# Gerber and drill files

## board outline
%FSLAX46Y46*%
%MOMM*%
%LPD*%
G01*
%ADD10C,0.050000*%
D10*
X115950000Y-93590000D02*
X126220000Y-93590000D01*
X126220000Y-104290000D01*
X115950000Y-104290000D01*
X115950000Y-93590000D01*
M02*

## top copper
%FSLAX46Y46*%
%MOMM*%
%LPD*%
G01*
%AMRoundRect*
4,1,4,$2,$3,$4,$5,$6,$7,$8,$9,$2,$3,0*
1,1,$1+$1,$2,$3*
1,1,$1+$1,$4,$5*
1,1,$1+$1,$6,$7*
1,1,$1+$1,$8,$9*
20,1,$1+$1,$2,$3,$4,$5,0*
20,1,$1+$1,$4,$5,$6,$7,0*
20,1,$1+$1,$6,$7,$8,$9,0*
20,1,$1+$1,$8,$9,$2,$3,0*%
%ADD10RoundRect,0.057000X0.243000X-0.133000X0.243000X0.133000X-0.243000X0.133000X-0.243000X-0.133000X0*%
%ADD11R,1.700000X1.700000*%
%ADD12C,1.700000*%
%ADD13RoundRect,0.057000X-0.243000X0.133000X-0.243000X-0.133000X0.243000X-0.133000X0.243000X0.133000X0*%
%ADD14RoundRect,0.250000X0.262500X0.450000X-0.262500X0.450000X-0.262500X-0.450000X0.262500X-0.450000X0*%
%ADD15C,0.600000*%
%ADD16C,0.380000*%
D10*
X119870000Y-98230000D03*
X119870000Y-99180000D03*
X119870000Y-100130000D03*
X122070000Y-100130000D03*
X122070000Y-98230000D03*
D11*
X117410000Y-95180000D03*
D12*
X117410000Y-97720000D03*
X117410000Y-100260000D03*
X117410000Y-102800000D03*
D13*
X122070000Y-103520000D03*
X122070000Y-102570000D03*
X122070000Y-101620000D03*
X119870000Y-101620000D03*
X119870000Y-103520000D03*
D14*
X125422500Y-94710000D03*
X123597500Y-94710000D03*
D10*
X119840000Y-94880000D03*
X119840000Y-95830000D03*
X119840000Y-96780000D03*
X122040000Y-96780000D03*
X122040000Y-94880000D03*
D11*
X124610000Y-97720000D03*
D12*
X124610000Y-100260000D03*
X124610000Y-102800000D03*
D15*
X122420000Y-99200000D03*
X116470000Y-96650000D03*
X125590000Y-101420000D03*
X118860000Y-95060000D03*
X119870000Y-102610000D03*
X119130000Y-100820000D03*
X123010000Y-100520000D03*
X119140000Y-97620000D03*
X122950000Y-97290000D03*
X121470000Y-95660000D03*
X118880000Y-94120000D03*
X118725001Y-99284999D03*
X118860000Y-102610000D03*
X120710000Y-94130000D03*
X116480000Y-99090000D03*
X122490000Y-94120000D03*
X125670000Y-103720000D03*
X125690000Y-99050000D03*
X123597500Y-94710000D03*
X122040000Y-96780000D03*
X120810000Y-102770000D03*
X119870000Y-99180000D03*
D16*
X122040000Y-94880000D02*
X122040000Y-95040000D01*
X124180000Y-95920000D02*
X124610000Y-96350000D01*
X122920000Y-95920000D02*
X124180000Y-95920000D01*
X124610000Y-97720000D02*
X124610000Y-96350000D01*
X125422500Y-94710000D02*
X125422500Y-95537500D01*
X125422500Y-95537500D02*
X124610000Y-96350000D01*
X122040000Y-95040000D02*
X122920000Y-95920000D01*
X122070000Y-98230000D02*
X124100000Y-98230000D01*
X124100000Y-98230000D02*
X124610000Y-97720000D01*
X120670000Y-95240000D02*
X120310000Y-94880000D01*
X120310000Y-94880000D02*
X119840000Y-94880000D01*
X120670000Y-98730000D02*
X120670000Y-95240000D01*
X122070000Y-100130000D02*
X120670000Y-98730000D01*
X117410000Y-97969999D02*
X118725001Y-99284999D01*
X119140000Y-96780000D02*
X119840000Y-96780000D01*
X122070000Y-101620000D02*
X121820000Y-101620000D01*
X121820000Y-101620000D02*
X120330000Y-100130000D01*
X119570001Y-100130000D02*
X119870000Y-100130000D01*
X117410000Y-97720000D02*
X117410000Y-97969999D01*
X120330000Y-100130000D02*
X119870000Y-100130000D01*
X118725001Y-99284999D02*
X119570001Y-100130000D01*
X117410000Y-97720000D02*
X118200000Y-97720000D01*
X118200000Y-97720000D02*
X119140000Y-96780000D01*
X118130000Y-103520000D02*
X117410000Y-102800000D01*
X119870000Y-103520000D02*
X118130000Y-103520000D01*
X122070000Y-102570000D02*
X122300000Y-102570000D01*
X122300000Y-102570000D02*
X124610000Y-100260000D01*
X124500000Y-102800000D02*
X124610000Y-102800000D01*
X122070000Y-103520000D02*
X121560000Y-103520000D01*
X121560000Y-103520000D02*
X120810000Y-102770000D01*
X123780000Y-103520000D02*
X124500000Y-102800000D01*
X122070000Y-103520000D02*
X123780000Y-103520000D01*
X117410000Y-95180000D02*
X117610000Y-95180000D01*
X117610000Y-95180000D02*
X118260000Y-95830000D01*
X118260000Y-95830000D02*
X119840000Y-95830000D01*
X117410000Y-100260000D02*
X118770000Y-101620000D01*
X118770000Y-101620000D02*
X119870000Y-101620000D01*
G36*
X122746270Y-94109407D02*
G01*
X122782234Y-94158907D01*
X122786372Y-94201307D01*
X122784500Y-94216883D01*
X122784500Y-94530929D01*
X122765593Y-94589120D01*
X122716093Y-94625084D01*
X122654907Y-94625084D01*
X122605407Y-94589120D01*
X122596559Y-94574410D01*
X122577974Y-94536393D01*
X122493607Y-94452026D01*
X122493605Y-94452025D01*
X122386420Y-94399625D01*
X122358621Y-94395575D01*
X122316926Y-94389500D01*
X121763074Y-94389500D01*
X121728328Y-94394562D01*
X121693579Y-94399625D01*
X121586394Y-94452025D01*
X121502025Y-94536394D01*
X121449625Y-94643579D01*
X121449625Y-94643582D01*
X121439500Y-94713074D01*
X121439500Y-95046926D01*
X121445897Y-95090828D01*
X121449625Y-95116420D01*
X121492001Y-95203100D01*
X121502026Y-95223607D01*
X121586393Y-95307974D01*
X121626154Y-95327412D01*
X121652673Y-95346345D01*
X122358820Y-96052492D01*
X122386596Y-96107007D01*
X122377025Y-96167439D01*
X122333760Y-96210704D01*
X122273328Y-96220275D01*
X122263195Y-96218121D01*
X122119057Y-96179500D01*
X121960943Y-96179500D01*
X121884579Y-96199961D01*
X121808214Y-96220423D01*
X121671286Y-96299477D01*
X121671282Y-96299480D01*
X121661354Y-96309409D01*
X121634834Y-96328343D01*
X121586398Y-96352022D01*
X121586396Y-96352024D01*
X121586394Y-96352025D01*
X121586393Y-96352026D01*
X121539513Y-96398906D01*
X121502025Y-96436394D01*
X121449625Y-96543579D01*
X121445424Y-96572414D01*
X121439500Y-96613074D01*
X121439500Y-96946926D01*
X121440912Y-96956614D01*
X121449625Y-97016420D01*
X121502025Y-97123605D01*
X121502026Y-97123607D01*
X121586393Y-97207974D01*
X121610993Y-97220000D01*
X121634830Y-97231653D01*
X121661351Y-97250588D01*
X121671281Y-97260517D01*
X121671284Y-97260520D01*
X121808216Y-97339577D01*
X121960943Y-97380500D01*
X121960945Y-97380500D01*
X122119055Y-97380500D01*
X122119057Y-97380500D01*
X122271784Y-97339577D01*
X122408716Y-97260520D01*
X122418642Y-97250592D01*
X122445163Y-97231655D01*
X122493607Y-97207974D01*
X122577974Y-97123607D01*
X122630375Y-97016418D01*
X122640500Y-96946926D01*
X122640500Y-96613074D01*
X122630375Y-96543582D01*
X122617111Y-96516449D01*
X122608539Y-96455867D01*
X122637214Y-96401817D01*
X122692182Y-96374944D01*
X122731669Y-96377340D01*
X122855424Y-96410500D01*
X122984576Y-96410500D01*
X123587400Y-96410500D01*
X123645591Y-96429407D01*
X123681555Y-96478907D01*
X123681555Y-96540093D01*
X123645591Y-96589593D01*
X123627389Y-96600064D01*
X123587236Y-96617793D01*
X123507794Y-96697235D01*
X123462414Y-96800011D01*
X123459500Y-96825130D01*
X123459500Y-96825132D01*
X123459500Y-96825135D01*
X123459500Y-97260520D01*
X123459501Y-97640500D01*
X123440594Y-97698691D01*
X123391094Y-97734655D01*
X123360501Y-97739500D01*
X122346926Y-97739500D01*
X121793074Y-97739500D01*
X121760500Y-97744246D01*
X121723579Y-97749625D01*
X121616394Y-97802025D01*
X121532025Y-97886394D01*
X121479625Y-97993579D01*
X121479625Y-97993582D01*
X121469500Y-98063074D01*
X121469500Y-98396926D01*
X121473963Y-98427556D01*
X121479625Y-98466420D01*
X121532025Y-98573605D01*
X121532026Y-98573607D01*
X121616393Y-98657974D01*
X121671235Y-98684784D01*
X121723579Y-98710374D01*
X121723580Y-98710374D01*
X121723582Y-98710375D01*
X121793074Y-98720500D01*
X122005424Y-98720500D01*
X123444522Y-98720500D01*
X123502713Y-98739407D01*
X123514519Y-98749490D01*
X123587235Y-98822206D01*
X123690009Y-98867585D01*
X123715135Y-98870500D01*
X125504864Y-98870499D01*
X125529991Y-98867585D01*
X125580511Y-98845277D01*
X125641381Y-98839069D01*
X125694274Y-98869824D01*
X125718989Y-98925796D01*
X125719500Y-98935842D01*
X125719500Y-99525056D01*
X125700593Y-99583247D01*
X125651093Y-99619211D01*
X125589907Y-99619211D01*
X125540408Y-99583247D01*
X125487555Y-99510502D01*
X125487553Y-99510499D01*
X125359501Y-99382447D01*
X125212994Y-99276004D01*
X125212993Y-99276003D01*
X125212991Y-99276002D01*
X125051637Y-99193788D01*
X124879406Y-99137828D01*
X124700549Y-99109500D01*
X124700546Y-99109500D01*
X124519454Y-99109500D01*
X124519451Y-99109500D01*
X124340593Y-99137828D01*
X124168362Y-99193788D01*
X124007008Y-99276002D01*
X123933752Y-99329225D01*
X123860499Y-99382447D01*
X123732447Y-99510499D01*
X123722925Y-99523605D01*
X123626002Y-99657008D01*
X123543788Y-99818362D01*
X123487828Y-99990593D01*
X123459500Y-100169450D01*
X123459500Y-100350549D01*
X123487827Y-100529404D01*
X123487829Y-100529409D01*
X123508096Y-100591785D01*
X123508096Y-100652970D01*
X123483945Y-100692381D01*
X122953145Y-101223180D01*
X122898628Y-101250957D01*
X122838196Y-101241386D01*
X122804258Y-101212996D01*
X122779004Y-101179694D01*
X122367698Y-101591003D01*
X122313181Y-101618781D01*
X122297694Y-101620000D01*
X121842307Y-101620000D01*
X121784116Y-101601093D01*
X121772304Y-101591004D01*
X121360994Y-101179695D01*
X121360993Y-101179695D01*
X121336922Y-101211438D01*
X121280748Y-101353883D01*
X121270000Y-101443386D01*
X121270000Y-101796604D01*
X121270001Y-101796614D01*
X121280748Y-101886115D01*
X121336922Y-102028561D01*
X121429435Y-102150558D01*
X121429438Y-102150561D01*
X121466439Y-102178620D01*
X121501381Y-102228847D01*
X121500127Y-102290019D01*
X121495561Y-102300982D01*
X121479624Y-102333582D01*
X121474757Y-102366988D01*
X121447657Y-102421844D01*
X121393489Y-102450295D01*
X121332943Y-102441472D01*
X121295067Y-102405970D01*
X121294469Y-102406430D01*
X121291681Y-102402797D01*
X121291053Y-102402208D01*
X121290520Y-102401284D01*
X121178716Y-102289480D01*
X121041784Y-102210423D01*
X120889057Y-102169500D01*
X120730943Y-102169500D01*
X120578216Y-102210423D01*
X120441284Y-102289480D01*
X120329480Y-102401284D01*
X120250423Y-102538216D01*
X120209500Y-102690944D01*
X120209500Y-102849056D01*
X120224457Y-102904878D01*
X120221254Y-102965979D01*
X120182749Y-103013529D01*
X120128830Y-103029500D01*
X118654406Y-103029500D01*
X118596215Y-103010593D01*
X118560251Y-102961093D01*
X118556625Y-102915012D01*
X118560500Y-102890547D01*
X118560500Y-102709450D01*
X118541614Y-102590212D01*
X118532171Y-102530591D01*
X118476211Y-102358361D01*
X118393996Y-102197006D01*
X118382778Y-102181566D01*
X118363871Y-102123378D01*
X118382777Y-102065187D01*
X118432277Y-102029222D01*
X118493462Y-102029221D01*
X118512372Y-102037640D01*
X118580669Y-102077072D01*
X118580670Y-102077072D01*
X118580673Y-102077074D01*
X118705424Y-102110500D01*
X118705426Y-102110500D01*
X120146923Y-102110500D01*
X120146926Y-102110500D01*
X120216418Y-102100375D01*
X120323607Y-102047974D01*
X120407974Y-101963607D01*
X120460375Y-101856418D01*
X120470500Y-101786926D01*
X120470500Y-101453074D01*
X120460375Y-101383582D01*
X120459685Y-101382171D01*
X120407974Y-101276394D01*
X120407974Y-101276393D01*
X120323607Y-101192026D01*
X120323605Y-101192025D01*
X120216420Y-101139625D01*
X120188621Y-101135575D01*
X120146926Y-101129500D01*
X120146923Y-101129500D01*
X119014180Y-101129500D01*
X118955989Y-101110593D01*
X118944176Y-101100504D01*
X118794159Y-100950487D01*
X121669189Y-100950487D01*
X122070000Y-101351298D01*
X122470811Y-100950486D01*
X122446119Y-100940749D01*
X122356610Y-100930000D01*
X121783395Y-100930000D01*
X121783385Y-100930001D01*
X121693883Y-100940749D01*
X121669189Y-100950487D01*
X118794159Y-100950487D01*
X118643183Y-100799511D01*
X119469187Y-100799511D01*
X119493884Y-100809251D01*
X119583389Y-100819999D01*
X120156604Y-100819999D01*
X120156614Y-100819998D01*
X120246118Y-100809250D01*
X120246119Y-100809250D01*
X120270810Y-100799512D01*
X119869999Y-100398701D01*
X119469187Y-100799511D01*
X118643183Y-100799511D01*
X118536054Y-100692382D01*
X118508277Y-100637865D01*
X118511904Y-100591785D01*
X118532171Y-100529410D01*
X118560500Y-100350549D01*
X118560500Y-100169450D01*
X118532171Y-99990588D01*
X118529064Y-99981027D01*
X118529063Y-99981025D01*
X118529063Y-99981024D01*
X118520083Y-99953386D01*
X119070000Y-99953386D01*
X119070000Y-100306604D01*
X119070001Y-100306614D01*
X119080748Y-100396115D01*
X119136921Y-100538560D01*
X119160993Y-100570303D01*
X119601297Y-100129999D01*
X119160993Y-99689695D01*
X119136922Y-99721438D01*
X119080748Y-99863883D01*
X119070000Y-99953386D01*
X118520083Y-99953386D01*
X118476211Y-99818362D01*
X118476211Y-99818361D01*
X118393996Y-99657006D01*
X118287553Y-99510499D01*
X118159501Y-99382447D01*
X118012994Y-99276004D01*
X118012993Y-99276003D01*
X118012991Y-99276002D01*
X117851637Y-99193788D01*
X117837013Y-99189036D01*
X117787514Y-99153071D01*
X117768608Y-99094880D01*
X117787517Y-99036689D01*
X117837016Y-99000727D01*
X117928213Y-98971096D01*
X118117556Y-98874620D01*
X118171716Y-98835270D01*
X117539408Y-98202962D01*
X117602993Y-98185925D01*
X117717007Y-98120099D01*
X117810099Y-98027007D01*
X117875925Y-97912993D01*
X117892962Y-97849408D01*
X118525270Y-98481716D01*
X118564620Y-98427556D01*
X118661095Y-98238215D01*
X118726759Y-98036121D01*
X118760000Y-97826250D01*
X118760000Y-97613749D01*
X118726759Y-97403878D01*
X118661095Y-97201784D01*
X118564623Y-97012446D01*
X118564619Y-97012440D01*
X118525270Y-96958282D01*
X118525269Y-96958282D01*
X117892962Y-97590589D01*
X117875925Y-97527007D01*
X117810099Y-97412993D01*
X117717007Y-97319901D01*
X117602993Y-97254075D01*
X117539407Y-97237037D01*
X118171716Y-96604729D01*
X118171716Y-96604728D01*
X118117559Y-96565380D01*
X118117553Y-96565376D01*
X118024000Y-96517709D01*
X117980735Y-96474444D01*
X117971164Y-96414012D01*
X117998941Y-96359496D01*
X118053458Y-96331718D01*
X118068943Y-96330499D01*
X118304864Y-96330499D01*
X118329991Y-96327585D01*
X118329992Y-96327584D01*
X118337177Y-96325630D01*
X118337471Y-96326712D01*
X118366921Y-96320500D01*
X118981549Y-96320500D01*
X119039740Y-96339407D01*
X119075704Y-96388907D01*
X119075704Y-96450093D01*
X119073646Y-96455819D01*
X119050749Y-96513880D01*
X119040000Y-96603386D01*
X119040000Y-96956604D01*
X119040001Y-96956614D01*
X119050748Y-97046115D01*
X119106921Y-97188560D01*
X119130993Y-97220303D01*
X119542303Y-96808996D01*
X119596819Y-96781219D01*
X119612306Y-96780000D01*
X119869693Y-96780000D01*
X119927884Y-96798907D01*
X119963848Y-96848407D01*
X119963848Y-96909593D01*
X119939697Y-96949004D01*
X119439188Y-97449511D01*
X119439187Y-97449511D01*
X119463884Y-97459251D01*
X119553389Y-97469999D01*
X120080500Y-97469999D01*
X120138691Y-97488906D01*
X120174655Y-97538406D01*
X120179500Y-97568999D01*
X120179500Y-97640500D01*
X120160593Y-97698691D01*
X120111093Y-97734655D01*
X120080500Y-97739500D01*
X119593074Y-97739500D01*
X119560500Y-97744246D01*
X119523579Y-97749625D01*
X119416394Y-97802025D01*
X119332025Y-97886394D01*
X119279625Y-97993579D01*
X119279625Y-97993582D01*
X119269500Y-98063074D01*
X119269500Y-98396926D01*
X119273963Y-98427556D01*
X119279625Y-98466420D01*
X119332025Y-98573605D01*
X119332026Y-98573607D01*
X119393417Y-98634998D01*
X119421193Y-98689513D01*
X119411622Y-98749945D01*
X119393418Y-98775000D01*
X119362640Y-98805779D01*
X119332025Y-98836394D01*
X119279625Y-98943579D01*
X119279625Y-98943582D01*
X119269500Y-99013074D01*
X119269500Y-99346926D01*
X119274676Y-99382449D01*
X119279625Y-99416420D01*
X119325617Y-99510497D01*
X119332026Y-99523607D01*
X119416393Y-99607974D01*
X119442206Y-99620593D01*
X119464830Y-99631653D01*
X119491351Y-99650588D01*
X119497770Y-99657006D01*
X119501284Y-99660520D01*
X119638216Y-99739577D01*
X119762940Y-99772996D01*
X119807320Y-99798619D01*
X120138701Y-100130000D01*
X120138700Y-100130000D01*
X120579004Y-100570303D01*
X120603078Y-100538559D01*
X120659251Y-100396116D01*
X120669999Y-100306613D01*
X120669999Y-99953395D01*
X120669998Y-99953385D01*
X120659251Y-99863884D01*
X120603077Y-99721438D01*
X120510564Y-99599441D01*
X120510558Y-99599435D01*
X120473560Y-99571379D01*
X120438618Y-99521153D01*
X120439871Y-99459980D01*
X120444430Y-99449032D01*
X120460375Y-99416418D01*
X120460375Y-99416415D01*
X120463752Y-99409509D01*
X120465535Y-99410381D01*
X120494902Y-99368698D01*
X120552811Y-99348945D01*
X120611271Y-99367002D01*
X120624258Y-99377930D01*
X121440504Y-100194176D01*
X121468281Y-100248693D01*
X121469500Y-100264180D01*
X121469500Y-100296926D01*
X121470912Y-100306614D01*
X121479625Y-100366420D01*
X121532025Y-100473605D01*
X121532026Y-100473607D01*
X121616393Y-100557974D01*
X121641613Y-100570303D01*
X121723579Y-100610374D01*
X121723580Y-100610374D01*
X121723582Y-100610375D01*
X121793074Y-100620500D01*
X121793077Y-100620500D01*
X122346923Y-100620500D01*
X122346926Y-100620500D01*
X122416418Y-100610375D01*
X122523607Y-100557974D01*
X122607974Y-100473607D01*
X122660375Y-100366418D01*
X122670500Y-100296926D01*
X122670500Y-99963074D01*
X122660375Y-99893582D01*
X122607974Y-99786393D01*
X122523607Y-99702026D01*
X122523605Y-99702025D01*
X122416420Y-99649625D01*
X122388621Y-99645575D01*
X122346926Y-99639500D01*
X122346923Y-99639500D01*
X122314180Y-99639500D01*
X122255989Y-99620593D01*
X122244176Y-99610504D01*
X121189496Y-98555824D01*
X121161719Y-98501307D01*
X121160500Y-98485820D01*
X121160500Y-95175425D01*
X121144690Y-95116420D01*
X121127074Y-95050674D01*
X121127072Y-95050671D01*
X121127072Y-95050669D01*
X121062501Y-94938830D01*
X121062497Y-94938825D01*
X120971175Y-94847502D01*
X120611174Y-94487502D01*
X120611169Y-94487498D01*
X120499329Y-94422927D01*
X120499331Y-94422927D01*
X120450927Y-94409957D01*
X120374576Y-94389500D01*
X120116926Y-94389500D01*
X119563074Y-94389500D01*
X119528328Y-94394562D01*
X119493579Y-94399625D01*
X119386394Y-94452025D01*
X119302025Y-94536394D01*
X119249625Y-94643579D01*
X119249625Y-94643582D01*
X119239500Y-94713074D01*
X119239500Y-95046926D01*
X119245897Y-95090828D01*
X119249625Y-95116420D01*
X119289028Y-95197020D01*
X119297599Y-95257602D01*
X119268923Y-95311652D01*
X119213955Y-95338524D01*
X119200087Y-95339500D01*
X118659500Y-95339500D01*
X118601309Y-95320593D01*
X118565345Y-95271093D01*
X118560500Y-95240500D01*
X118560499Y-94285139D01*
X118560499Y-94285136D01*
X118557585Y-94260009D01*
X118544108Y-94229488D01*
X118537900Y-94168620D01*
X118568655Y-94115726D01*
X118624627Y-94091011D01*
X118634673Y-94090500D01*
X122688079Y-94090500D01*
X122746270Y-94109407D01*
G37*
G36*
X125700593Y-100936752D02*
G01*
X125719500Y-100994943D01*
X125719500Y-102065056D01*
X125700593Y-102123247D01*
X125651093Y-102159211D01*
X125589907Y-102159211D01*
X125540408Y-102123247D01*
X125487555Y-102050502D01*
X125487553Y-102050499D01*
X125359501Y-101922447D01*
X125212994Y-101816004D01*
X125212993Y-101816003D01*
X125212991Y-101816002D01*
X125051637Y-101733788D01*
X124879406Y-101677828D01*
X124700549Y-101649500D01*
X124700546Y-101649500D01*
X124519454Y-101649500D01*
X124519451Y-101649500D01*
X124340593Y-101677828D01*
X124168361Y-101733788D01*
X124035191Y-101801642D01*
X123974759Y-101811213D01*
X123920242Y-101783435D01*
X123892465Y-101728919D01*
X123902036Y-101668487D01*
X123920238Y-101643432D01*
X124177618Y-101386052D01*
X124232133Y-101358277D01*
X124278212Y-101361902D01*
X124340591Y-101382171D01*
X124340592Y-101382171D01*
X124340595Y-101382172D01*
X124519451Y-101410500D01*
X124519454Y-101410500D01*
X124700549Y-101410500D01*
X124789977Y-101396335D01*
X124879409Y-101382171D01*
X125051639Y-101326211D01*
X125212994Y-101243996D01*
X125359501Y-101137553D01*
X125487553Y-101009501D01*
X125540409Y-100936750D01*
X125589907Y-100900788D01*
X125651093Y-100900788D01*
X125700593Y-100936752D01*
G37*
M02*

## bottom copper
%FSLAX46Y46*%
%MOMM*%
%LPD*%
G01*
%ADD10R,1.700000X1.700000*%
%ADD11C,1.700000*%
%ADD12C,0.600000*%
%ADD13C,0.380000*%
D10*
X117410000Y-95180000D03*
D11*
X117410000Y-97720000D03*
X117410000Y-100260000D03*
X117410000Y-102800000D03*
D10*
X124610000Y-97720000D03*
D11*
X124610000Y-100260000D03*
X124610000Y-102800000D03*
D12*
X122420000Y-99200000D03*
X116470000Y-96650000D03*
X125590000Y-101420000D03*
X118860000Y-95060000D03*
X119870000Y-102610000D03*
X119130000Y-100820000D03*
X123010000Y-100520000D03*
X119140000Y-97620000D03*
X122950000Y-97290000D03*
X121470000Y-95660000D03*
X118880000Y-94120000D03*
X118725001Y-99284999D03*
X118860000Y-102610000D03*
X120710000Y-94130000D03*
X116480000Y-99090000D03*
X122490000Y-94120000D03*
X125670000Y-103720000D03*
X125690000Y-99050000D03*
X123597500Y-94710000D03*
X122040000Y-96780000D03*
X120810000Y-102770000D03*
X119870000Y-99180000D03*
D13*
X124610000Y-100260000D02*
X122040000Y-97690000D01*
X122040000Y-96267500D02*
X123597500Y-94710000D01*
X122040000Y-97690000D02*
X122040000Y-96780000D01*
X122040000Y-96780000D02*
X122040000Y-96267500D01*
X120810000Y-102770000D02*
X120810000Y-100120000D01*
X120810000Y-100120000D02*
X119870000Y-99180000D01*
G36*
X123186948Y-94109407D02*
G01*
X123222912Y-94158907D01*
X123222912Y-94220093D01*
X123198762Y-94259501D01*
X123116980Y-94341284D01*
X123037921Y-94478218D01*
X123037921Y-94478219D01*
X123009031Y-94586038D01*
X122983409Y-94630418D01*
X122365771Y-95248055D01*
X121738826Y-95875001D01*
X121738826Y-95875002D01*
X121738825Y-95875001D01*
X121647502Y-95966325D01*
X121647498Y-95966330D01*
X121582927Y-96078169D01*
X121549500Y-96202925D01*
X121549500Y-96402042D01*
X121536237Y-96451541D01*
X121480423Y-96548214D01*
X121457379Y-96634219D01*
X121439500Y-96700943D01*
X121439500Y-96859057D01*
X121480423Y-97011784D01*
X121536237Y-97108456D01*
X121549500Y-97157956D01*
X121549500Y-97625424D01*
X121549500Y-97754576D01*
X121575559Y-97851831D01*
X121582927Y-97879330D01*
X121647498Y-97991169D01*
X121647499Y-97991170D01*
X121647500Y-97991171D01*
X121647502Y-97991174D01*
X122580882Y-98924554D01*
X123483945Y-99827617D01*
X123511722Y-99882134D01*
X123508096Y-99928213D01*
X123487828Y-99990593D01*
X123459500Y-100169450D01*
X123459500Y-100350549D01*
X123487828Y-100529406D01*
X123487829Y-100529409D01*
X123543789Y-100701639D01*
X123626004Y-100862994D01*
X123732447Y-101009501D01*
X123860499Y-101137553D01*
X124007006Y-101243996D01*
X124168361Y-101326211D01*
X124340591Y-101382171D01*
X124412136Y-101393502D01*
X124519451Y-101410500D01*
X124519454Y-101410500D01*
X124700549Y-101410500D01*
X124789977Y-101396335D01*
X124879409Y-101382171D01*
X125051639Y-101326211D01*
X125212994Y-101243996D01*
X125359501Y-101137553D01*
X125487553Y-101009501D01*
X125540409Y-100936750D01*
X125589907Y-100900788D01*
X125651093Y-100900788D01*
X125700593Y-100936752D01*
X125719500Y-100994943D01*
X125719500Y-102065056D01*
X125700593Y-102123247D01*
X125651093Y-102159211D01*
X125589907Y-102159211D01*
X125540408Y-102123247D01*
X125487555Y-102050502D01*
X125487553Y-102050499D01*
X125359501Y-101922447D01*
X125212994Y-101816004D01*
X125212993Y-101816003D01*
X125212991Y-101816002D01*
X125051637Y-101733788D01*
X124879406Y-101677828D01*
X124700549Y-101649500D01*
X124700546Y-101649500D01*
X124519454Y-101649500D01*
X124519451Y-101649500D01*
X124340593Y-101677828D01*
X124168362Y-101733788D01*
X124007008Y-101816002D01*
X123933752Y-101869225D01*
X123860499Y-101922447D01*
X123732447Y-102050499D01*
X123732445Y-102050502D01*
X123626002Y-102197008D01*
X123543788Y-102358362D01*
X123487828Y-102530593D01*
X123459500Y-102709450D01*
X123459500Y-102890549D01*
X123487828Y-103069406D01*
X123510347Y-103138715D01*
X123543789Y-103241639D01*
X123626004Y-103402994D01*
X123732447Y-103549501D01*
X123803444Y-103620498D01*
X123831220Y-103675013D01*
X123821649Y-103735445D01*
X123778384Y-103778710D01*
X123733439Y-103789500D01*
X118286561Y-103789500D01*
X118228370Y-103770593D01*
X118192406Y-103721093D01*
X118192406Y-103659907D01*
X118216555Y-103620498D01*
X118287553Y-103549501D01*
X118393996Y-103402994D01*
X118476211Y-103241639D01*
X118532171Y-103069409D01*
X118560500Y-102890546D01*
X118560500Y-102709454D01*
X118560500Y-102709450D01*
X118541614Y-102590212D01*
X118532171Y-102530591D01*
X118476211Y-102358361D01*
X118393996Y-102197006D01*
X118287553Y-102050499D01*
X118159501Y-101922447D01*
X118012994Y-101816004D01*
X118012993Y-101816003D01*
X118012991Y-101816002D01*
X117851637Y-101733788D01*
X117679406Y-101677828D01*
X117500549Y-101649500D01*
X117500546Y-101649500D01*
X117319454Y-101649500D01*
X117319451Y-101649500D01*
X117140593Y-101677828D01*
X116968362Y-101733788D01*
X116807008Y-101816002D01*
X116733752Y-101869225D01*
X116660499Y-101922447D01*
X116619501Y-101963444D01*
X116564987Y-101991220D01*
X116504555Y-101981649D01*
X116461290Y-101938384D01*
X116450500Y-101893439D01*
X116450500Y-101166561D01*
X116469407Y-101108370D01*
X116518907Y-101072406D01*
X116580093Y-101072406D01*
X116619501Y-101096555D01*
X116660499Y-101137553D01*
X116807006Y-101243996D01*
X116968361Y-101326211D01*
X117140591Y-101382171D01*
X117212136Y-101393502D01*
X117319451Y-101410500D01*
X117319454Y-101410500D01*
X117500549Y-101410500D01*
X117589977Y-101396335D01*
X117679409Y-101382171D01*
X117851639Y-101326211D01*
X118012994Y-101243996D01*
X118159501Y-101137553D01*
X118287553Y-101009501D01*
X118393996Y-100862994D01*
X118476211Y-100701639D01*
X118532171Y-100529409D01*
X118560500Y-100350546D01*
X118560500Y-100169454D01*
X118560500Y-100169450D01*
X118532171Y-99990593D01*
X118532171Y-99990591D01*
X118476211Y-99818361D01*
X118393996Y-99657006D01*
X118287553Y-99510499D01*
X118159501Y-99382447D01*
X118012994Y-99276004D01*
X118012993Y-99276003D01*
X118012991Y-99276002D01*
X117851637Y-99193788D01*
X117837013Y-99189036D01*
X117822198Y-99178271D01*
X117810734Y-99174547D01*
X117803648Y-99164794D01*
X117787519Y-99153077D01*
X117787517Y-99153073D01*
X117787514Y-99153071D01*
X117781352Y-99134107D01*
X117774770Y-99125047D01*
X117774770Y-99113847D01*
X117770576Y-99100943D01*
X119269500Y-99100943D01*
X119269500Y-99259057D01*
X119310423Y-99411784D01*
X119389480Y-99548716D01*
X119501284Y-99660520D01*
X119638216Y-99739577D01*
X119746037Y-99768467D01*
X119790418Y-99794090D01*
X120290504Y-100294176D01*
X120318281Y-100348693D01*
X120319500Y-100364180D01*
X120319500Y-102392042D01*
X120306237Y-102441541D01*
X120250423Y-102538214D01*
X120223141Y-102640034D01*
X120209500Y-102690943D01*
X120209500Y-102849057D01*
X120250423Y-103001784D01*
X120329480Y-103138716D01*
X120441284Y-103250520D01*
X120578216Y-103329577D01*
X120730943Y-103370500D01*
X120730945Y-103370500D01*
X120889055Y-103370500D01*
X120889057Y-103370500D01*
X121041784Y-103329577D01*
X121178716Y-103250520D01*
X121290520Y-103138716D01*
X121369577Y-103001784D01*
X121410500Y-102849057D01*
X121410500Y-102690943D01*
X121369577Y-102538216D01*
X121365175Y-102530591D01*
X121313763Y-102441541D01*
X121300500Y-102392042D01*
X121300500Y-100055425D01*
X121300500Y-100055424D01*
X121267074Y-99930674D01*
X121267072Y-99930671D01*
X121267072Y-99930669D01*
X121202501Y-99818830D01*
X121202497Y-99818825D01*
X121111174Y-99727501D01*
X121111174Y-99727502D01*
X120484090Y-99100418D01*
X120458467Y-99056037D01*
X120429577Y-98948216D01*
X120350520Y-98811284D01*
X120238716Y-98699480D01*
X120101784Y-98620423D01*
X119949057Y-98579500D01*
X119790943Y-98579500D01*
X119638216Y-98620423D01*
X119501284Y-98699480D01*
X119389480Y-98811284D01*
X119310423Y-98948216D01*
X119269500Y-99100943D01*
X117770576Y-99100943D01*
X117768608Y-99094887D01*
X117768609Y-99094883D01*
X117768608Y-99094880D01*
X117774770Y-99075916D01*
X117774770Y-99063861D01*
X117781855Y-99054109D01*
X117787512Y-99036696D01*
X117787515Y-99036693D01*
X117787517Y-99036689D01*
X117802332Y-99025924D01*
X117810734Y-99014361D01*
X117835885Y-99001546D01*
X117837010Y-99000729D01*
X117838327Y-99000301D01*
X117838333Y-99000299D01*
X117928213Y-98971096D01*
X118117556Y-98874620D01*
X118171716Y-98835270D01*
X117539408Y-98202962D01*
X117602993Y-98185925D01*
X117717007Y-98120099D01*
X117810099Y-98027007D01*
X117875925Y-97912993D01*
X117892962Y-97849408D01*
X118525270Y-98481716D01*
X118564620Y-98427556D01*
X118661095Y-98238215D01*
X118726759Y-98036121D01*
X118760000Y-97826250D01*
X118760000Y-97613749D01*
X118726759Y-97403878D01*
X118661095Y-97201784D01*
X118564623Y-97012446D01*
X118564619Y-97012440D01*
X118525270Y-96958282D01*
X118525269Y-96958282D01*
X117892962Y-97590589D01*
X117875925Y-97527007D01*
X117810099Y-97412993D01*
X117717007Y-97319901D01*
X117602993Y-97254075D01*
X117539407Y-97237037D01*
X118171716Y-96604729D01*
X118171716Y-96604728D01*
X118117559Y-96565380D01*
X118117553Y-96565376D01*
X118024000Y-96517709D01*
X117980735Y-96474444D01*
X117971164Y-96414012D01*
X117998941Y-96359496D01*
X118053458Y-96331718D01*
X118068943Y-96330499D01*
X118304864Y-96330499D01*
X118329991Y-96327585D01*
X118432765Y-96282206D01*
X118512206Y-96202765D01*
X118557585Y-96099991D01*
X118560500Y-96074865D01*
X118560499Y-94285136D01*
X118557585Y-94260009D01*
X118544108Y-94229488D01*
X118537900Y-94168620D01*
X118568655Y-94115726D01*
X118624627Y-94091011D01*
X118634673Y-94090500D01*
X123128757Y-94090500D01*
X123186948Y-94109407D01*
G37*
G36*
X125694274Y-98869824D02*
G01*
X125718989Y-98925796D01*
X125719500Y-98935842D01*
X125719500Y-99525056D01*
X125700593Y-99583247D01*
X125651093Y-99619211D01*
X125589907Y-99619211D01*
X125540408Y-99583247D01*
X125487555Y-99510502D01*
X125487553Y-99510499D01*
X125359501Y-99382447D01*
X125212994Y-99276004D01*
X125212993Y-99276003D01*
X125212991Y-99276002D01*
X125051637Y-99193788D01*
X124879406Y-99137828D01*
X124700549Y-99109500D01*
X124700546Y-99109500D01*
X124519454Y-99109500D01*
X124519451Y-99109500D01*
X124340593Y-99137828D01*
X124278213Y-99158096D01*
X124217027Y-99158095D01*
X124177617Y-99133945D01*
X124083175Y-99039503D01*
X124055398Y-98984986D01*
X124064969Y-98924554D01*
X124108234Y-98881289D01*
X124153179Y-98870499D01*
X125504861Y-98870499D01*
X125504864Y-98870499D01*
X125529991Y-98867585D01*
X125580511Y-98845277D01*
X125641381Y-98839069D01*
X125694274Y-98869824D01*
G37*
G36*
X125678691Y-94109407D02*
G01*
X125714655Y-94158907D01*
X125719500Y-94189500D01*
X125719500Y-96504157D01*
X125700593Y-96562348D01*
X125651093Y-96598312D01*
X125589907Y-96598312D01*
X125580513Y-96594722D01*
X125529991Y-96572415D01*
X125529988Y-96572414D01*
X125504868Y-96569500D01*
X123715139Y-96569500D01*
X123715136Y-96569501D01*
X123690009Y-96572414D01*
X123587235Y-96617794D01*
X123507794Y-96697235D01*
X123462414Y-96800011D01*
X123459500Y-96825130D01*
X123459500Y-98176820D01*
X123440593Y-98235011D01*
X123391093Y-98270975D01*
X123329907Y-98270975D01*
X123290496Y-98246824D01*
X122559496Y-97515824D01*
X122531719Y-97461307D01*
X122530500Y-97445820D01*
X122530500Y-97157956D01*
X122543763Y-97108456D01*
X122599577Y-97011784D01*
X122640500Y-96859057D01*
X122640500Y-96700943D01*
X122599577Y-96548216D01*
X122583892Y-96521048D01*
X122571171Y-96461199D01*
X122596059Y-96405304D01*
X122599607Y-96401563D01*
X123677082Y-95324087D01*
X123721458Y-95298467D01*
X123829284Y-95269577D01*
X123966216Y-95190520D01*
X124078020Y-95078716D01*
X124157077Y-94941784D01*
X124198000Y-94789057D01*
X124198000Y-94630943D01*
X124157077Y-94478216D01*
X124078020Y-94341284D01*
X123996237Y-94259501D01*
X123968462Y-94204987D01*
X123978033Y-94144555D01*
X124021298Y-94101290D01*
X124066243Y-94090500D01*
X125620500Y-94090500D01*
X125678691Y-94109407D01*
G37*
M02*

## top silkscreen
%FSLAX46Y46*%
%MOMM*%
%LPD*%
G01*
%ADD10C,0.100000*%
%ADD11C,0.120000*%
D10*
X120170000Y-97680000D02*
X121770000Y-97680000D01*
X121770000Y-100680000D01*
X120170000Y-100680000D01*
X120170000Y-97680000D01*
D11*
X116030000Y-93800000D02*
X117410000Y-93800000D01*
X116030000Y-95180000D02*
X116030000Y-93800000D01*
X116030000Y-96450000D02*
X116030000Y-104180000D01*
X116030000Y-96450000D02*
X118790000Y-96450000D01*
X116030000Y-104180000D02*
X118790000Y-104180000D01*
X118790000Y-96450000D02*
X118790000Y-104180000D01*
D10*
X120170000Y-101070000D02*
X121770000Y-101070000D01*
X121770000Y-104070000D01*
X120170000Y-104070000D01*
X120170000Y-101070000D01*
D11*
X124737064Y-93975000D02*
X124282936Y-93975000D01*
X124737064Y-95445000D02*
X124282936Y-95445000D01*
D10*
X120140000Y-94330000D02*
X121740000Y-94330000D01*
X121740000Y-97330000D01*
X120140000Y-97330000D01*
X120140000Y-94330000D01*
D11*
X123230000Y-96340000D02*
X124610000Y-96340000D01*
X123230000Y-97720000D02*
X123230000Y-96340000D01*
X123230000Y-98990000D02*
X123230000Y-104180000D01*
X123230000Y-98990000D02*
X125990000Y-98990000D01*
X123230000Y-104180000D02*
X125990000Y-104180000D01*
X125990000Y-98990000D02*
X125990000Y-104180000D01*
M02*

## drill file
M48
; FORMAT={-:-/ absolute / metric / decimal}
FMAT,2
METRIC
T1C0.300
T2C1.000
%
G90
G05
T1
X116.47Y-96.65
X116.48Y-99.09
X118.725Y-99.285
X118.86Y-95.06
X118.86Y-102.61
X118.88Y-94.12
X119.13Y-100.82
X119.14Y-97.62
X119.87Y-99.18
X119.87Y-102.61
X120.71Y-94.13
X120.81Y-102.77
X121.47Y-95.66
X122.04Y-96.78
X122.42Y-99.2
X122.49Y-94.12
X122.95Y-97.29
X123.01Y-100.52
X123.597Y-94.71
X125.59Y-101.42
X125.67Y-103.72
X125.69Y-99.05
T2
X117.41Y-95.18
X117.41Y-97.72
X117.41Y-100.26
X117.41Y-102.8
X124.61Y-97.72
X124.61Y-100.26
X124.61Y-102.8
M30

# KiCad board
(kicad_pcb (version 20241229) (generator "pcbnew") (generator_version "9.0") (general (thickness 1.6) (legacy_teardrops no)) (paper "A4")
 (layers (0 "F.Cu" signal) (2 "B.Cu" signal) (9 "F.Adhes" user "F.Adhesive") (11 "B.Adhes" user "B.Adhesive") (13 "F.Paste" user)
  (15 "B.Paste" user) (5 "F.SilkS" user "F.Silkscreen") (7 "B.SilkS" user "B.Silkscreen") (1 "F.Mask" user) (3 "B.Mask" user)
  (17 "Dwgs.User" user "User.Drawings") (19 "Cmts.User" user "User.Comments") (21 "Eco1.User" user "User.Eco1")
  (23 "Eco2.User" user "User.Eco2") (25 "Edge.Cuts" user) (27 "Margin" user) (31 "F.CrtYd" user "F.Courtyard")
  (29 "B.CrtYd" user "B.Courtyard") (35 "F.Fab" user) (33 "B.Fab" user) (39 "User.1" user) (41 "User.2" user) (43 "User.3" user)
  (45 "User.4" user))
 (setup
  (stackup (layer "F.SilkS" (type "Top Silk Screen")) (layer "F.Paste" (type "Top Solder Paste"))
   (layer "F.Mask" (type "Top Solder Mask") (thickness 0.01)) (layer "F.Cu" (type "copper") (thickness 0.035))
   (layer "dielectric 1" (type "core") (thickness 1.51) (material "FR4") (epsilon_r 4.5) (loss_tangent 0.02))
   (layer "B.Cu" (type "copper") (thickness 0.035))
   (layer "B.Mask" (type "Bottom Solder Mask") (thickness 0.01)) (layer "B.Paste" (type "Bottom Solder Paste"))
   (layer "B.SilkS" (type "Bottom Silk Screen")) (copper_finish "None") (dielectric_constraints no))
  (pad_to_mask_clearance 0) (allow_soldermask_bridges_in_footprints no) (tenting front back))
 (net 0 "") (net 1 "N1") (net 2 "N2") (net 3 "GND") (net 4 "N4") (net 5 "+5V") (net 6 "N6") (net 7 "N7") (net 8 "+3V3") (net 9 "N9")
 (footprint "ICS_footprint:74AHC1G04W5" (layer "F.Cu") (at 120.97 99.18 90)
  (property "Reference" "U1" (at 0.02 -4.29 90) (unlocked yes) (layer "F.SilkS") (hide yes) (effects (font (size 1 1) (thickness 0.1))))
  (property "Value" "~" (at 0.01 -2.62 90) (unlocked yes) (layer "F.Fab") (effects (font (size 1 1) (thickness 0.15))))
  (fp_rect (start -1.5 -0.8) (end 1.5 0.8) (stroke (width 0.1) (type solid)) (fill no) (layer "F.SilkS"))
  (pad "1" smd roundrect (at 0.95 -1.1 90) (size 0.38 0.6) (layers "F.Cu" "F.Mask" "F.Paste") (roundrect_rratio 0.15) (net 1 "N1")
   (thermal_bridge_angle 45))
  (pad "2" smd roundrect (at 0 -1.1 90) (size 0.38 0.6) (layers "F.Cu" "F.Mask" "F.Paste") (roundrect_rratio 0.15) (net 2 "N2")
   (thermal_bridge_angle 45))
  (pad "3" smd roundrect (at -0.95 -1.1 90) (size 0.38 0.6) (layers "F.Cu" "F.Mask" "F.Paste") (roundrect_rratio 0.15) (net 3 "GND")
   (thermal_bridge_angle 45))
  (pad "4" smd roundrect (at -0.95 1.1 90) (size 0.38 0.6) (layers "F.Cu" "F.Mask" "F.Paste") (roundrect_rratio 0.15) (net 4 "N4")
   (thermal_bridge_angle 45))
  (pad "5" smd roundrect (at 0.95 1.1 90) (size 0.38 0.6) (layers "F.Cu" "F.Mask" "F.Paste") (roundrect_rratio 0.15) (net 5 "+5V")
   (thermal_bridge_angle 45)))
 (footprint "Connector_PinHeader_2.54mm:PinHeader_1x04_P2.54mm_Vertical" (layer "F.Cu") (at 117.41 95.18)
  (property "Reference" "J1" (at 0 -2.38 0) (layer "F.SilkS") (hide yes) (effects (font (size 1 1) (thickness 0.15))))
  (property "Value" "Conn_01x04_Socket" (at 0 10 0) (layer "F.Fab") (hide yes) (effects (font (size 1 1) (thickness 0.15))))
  (fp_line (start -1.38 -1.38) (end 0 -1.38) (stroke (width 0.12) (type solid)) (layer "F.SilkS"))
  (fp_line (start -1.38 0) (end -1.38 -1.38) (stroke (width 0.12) (type solid)) (layer "F.SilkS"))
  (fp_line (start -1.38 1.27) (end -1.38 9) (stroke (width 0.12) (type solid)) (layer "F.SilkS"))
  (fp_line (start -1.38 1.27) (end 1.38 1.27) (stroke (width 0.12) (type solid)) (layer "F.SilkS"))
  (fp_line (start -1.38 9) (end 1.38 9) (stroke (width 0.12) (type solid)) (layer "F.SilkS"))
  (fp_line (start 1.38 1.27) (end 1.38 9) (stroke (width 0.12) (type solid)) (layer "F.SilkS"))
  (pad "1" thru_hole rect (at 0 0) (size 1.7 1.7) (drill 1) (layers "*.Cu" "*.Mask") (remove_unused_layers no) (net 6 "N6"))
  (pad "2" thru_hole circle (at 0 2.54) (size 1.7 1.7) (drill 1) (layers "*.Cu" "*.Mask") (remove_unused_layers no) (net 3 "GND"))
  (pad "3" thru_hole circle (at 0 5.08) (size 1.7 1.7) (drill 1) (layers "*.Cu" "*.Mask") (remove_unused_layers no) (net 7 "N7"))
  (pad "4" thru_hole circle (at 0 7.62) (size 1.7 1.7) (drill 1) (layers "*.Cu" "*.Mask") (remove_unused_layers no) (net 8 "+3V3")))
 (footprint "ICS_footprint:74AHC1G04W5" (layer "F.Cu") (at 120.97 102.57 -90)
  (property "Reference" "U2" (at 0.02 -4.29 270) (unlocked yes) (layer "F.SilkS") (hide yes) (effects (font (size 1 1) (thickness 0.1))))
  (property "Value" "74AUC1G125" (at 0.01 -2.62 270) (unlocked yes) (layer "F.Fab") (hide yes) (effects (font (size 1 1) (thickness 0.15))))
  (fp_rect (start -1.5 -0.8) (end 1.5 0.8) (stroke (width 0.1) (type solid)) (fill no) (layer "F.SilkS"))
  (pad "1" smd roundrect (at 0.95 -1.1 270) (size 0.38 0.6) (layers "F.Cu" "F.Mask" "F.Paste") (roundrect_rratio 0.15) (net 2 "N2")
   (thermal_bridge_angle 45))
  (pad "2" smd roundrect (at 0 -1.1 270) (size 0.38 0.6) (layers "F.Cu" "F.Mask" "F.Paste") (roundrect_rratio 0.15) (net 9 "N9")
   (thermal_bridge_angle 45))
  (pad "3" smd roundrect (at -0.95 -1.1 270) (size 0.38 0.6) (layers "F.Cu" "F.Mask" "F.Paste") (roundrect_rratio 0.15) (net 3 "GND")
   (thermal_bridge_angle 45))
  (pad "4" smd roundrect (at -0.95 1.1 270) (size 0.38 0.6) (layers "F.Cu" "F.Mask" "F.Paste") (roundrect_rratio 0.15) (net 7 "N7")
   (thermal_bridge_angle 45))
  (pad "5" smd roundrect (at 0.95 1.1 270) (size 0.38 0.6) (layers "F.Cu" "F.Mask" "F.Paste") (roundrect_rratio 0.15) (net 8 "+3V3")
   (thermal_bridge_angle 45)))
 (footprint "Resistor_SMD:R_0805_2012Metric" (layer "F.Cu") (at 124.51 94.71 180)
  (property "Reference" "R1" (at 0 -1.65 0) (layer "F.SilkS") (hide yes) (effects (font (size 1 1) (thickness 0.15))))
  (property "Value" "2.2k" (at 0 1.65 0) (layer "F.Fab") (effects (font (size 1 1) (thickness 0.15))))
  (fp_line (start -0.227064 0.735) (end 0.227064 0.735) (stroke (width 0.12) (type solid)) (layer "F.SilkS"))
  (fp_line (start -0.227064 -0.735) (end 0.227064 -0.735) (stroke (width 0.12) (type solid)) (layer "F.SilkS"))
  (pad "1" smd roundrect (at -0.9125 0 180) (size 1.025 1.4) (layers "F.Cu" "F.Mask" "F.Paste") (roundrect_rratio 0.243902) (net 5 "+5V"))
  (pad "2" smd roundrect (at 0.9125 0 180) (size 1.025 1.4) (layers "F.Cu" "F.Mask" "F.Paste") (roundrect_rratio 0.243902) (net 9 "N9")))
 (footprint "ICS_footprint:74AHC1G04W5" (layer "F.Cu") (at 120.94 95.83 90)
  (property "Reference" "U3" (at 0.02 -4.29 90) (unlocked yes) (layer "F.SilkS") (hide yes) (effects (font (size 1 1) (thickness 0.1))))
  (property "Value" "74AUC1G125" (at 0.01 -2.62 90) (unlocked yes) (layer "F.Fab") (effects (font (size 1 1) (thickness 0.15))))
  (fp_rect (start -1.5 -0.8) (end 1.5 0.8) (stroke (width 0.1) (type solid)) (fill no) (layer "F.SilkS"))
  (pad "1" smd roundrect (at 0.95 -1.1 90) (size 0.38 0.6) (layers "F.Cu" "F.Mask" "F.Paste") (roundrect_rratio 0.15) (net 4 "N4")
   (thermal_bridge_angle 45))
  (pad "2" smd roundrect (at 0 -1.1 90) (size 0.38 0.6) (layers "F.Cu" "F.Mask" "F.Paste") (roundrect_rratio 0.15) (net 6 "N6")
   (thermal_bridge_angle 45))
  (pad "3" smd roundrect (at -0.95 -1.1 90) (size 0.38 0.6) (layers "F.Cu" "F.Mask" "F.Paste") (roundrect_rratio 0.15) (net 3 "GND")
   (thermal_bridge_angle 45))
  (pad "4" smd roundrect (at -0.95 1.1 90) (size 0.38 0.6) (layers "F.Cu" "F.Mask" "F.Paste") (roundrect_rratio 0.15) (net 9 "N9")
   (thermal_bridge_angle 45))
  (pad "5" smd roundrect (at 0.95 1.1 90) (size 0.38 0.6) (layers "F.Cu" "F.Mask" "F.Paste") (roundrect_rratio 0.15) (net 5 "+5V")
   (thermal_bridge_angle 45)))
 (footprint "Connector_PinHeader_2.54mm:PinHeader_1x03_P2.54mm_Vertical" (layer "F.Cu") (at 124.61 97.72)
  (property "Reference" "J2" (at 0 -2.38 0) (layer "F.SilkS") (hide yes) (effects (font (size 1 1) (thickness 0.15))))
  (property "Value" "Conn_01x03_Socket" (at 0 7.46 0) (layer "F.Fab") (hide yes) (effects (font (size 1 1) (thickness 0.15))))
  (fp_line (start -1.38 -1.38) (end 0 -1.38) (stroke (width 0.12) (type solid)) (layer "F.SilkS"))
  (fp_line (start -1.38 0) (end -1.38 -1.38) (stroke (width 0.12) (type solid)) (layer "F.SilkS"))
  (fp_line (start -1.38 1.27) (end -1.38 6.46) (stroke (width 0.12) (type solid)) (layer "F.SilkS"))
  (fp_line (start -1.38 1.27) (end 1.38 1.27) (stroke (width 0.12) (type solid)) (layer "F.SilkS"))
  (fp_line (start -1.38 6.46) (end 1.38 6.46) (stroke (width 0.12) (type solid)) (layer "F.SilkS"))
  (fp_line (start 1.38 1.27) (end 1.38 6.46) (stroke (width 0.12) (type solid)) (layer "F.SilkS"))
  (pad "1" thru_hole rect (at 0 0) (size 1.7 1.7) (drill 1) (layers "*.Cu" "*.Mask") (remove_unused_layers no) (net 5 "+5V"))
  (pad "2" thru_hole circle (at 0 2.54) (size 1.7 1.7) (drill 1) (layers "*.Cu" "*.Mask") (remove_unused_layers no) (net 9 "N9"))
  (pad "3" thru_hole circle (at 0 5.08) (size 1.7 1.7) (drill 1) (layers "*.Cu" "*.Mask") (remove_unused_layers no) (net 2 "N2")))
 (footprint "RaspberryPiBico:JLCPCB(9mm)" (layer "B.Cu") (at 121.22467 98.45426 115)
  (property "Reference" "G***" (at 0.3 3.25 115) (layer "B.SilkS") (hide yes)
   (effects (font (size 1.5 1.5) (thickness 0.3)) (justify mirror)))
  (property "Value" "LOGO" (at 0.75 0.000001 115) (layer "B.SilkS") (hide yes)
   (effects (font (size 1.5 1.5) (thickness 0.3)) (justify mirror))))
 (gr_rect (start 115.95 93.59) (end 126.22 104.29) (stroke (width 0.05) (type default)) (fill no) (layer "Edge.Cuts"))
 (segment (start 122.04 94.88) (end 122.04 95.04) (width 0.38) (layer "F.Cu") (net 5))
 (segment (start 124.18 95.92) (end 124.61 96.35) (width 0.38) (layer "F.Cu") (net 5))
 (segment (start 122.92 95.92) (end 124.18 95.92) (width 0.38) (layer "F.Cu") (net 5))
 (segment (start 124.61 97.72) (end 124.61 96.35) (width 0.38) (layer "F.Cu") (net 5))
 (segment (start 125.4225 94.71) (end 125.4225 95.5375) (width 0.38) (layer "F.Cu") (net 5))
 (segment (start 125.4225 95.5375) (end 124.61 96.35) (width 0.38) (layer "F.Cu") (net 5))
 (segment (start 122.04 95.04) (end 122.92 95.92) (width 0.38) (layer "F.Cu") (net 5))
 (segment (start 122.07 98.23) (end 124.1 98.23) (width 0.38) (layer "F.Cu") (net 5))
 (segment (start 124.1 98.23) (end 124.61 97.72) (width 0.38) (layer "F.Cu") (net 5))
 (segment (start 120.67 95.24) (end 120.31 94.88) (width 0.38) (layer "F.Cu") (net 4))
 (segment (start 120.31 94.88) (end 119.84 94.88) (width 0.38) (layer "F.Cu") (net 4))
 (segment (start 120.67 98.73) (end 120.67 95.24) (width 0.38) (layer "F.Cu") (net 4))
 (segment (start 122.07 100.13) (end 120.67 98.73) (width 0.38) (layer "F.Cu") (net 4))
 (segment (start 117.41 97.969999) (end 118.725001 99.284999) (width 0.38) (layer "F.Cu") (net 3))
 (segment (start 119.14 96.78) (end 119.84 96.78) (width 0.38) (layer "F.Cu") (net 3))
 (segment (start 122.07 101.62) (end 121.82 101.62) (width 0.38) (layer "F.Cu") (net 3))
 (segment (start 121.82 101.62) (end 120.33 100.13) (width 0.38) (layer "F.Cu") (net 3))
 (segment (start 119.570001 100.13) (end 119.87 100.13) (width 0.38) (layer "F.Cu") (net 3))
 (segment (start 117.41 97.72) (end 117.41 97.969999) (width 0.38) (layer "F.Cu") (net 3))
 (segment (start 120.33 100.13) (end 119.87 100.13) (width 0.38) (layer "F.Cu") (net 3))
 (segment (start 118.725001 99.284999) (end 119.570001 100.13) (width 0.38) (layer "F.Cu") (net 3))
 (segment (start 117.41 97.72) (end 118.2 97.72) (width 0.38) (layer "F.Cu") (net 3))
 (segment (start 118.2 97.72) (end 119.14 96.78) (width 0.38) (layer "F.Cu") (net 3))
 (via (at 122.42 99.2) (size 0.6) (drill 0.3) (layers "F.Cu" "B.Cu") (free yes) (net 3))
 (via (at 116.47 96.65) (size 0.6) (drill 0.3) (layers "F.Cu" "B.Cu") (free yes) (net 3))
 (via (at 125.59 101.42) (size 0.6) (drill 0.3) (layers "F.Cu" "B.Cu") (free yes) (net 3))
 (via (at 118.86 95.06) (size 0.6) (drill 0.3) (layers "F.Cu" "B.Cu") (free yes) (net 3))
 (via (at 119.87 102.61) (size 0.6) (drill 0.3) (layers "F.Cu" "B.Cu") (free yes) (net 3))
 (via (at 119.13 100.82) (size 0.6) (drill 0.3) (layers "F.Cu" "B.Cu") (free yes) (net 3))
 (via (at 123.01 100.52) (size 0.6) (drill 0.3) (layers "F.Cu" "B.Cu") (free yes) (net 3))
 (via (at 119.14 97.62) (size 0.6) (drill 0.3) (layers "F.Cu" "B.Cu") (free yes) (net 3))
 (via (at 122.95 97.29) (size 0.6) (drill 0.3) (layers "F.Cu" "B.Cu") (free yes) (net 3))
 (via (at 121.47 95.66) (size 0.6) (drill 0.3) (layers "F.Cu" "B.Cu") (free yes) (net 3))
 (via (at 118.88 94.12) (size 0.6) (drill 0.3) (layers "F.Cu" "B.Cu") (free yes) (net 3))
 (via (at 118.725001 99.284999) (size 0.6) (drill 0.3) (layers "F.Cu" "B.Cu") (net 3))
 (via (at 118.86 102.61) (size 0.6) (drill 0.3) (layers "F.Cu" "B.Cu") (free yes) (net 3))
 (via (at 120.71 94.13) (size 0.6) (drill 0.3) (layers "F.Cu" "B.Cu") (free yes) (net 3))
 (via (at 116.48 99.09) (size 0.6) (drill 0.3) (layers "F.Cu" "B.Cu") (free yes) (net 3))
 (via (at 122.49 94.12) (size 0.6) (drill 0.3) (layers "F.Cu" "B.Cu") (free yes) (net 3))
 (via (at 125.67 103.72) (size 0.6) (drill 0.3) (layers "F.Cu" "B.Cu") (free yes) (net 3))
 (via (at 125.69 99.05) (size 0.6) (drill 0.3) (layers "F.Cu" "B.Cu") (free yes) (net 3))
 (segment (start 118.13 103.52) (end 117.41 102.8) (width 0.38) (layer "F.Cu") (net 8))
 (segment (start 119.87 103.52) (end 118.13 103.52) (width 0.38) (layer "F.Cu") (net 8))
 (segment (start 122.07 102.57) (end 122.3 102.57) (width 0.38) (layer "F.Cu") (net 9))
 (segment (start 122.3 102.57) (end 124.61 100.26) (width 0.38) (layer "F.Cu") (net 9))
 (via (at 123.5975 94.71) (size 0.6) (drill 0.3) (layers "F.Cu" "B.Cu") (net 9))
 (via (at 122.04 96.78) (size 0.6) (drill 0.3) (layers "F.Cu" "B.Cu") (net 9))
 (segment (start 124.61 100.26) (end 122.04 97.69) (width 0.38) (layer "B.Cu") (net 9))
 (segment (start 122.04 96.2675) (end 123.5975 94.71) (width 0.38) (layer "B.Cu") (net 9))
 (segment (start 122.04 97.69) (end 122.04 96.78) (width 0.38) (layer "B.Cu") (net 9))
 (segment (start 122.04 96.78) (end 122.04 96.2675) (width 0.38) (layer "B.Cu") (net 9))
 (segment (start 124.5 102.8) (end 124.61 102.8) (width 0.38) (layer "F.Cu") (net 2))
 (segment (start 122.07 103.52) (end 121.56 103.52) (width 0.38) (layer "F.Cu") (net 2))
 (segment (start 121.56 103.52) (end 120.81 102.77) (width 0.38) (layer "F.Cu") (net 2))
 (segment (start 123.78 103.52) (end 124.5 102.8) (width 0.38) (layer "F.Cu") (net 2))
 (segment (start 122.07 103.52) (end 123.78 103.52) (width 0.38) (layer "F.Cu") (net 2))
 (via (at 120.81 102.77) (size 0.6) (drill 0.3) (layers "F.Cu" "B.Cu") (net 2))
 (via (at 119.87 99.18) (size 0.6) (drill 0.3) (layers "F.Cu" "B.Cu") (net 2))
 (segment (start 120.81 102.77) (end 120.81 100.12) (width 0.38) (layer "B.Cu") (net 2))
 (segment (start 120.81 100.12) (end 119.87 99.18) (width 0.38) (layer "B.Cu") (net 2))
 (segment (start 117.41 95.18) (end 117.61 95.18) (width 0.38) (layer "F.Cu") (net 6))
 (segment (start 117.61 95.18) (end 118.26 95.83) (width 0.38) (layer "F.Cu") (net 6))
 (segment (start 118.26 95.83) (end 119.84 95.83) (width 0.38) (layer "F.Cu") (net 6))
 (segment (start 117.41 100.26) (end 118.77 101.62) (width 0.38) (layer "F.Cu") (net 7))
 (segment (start 118.77 101.62) (end 119.87 101.62) (width 0.38) (layer "F.Cu") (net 7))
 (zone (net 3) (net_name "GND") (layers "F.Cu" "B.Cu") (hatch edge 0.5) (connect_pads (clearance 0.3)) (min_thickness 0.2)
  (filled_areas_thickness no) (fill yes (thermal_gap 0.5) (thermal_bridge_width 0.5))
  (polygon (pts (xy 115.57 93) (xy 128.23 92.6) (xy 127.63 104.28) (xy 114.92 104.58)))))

